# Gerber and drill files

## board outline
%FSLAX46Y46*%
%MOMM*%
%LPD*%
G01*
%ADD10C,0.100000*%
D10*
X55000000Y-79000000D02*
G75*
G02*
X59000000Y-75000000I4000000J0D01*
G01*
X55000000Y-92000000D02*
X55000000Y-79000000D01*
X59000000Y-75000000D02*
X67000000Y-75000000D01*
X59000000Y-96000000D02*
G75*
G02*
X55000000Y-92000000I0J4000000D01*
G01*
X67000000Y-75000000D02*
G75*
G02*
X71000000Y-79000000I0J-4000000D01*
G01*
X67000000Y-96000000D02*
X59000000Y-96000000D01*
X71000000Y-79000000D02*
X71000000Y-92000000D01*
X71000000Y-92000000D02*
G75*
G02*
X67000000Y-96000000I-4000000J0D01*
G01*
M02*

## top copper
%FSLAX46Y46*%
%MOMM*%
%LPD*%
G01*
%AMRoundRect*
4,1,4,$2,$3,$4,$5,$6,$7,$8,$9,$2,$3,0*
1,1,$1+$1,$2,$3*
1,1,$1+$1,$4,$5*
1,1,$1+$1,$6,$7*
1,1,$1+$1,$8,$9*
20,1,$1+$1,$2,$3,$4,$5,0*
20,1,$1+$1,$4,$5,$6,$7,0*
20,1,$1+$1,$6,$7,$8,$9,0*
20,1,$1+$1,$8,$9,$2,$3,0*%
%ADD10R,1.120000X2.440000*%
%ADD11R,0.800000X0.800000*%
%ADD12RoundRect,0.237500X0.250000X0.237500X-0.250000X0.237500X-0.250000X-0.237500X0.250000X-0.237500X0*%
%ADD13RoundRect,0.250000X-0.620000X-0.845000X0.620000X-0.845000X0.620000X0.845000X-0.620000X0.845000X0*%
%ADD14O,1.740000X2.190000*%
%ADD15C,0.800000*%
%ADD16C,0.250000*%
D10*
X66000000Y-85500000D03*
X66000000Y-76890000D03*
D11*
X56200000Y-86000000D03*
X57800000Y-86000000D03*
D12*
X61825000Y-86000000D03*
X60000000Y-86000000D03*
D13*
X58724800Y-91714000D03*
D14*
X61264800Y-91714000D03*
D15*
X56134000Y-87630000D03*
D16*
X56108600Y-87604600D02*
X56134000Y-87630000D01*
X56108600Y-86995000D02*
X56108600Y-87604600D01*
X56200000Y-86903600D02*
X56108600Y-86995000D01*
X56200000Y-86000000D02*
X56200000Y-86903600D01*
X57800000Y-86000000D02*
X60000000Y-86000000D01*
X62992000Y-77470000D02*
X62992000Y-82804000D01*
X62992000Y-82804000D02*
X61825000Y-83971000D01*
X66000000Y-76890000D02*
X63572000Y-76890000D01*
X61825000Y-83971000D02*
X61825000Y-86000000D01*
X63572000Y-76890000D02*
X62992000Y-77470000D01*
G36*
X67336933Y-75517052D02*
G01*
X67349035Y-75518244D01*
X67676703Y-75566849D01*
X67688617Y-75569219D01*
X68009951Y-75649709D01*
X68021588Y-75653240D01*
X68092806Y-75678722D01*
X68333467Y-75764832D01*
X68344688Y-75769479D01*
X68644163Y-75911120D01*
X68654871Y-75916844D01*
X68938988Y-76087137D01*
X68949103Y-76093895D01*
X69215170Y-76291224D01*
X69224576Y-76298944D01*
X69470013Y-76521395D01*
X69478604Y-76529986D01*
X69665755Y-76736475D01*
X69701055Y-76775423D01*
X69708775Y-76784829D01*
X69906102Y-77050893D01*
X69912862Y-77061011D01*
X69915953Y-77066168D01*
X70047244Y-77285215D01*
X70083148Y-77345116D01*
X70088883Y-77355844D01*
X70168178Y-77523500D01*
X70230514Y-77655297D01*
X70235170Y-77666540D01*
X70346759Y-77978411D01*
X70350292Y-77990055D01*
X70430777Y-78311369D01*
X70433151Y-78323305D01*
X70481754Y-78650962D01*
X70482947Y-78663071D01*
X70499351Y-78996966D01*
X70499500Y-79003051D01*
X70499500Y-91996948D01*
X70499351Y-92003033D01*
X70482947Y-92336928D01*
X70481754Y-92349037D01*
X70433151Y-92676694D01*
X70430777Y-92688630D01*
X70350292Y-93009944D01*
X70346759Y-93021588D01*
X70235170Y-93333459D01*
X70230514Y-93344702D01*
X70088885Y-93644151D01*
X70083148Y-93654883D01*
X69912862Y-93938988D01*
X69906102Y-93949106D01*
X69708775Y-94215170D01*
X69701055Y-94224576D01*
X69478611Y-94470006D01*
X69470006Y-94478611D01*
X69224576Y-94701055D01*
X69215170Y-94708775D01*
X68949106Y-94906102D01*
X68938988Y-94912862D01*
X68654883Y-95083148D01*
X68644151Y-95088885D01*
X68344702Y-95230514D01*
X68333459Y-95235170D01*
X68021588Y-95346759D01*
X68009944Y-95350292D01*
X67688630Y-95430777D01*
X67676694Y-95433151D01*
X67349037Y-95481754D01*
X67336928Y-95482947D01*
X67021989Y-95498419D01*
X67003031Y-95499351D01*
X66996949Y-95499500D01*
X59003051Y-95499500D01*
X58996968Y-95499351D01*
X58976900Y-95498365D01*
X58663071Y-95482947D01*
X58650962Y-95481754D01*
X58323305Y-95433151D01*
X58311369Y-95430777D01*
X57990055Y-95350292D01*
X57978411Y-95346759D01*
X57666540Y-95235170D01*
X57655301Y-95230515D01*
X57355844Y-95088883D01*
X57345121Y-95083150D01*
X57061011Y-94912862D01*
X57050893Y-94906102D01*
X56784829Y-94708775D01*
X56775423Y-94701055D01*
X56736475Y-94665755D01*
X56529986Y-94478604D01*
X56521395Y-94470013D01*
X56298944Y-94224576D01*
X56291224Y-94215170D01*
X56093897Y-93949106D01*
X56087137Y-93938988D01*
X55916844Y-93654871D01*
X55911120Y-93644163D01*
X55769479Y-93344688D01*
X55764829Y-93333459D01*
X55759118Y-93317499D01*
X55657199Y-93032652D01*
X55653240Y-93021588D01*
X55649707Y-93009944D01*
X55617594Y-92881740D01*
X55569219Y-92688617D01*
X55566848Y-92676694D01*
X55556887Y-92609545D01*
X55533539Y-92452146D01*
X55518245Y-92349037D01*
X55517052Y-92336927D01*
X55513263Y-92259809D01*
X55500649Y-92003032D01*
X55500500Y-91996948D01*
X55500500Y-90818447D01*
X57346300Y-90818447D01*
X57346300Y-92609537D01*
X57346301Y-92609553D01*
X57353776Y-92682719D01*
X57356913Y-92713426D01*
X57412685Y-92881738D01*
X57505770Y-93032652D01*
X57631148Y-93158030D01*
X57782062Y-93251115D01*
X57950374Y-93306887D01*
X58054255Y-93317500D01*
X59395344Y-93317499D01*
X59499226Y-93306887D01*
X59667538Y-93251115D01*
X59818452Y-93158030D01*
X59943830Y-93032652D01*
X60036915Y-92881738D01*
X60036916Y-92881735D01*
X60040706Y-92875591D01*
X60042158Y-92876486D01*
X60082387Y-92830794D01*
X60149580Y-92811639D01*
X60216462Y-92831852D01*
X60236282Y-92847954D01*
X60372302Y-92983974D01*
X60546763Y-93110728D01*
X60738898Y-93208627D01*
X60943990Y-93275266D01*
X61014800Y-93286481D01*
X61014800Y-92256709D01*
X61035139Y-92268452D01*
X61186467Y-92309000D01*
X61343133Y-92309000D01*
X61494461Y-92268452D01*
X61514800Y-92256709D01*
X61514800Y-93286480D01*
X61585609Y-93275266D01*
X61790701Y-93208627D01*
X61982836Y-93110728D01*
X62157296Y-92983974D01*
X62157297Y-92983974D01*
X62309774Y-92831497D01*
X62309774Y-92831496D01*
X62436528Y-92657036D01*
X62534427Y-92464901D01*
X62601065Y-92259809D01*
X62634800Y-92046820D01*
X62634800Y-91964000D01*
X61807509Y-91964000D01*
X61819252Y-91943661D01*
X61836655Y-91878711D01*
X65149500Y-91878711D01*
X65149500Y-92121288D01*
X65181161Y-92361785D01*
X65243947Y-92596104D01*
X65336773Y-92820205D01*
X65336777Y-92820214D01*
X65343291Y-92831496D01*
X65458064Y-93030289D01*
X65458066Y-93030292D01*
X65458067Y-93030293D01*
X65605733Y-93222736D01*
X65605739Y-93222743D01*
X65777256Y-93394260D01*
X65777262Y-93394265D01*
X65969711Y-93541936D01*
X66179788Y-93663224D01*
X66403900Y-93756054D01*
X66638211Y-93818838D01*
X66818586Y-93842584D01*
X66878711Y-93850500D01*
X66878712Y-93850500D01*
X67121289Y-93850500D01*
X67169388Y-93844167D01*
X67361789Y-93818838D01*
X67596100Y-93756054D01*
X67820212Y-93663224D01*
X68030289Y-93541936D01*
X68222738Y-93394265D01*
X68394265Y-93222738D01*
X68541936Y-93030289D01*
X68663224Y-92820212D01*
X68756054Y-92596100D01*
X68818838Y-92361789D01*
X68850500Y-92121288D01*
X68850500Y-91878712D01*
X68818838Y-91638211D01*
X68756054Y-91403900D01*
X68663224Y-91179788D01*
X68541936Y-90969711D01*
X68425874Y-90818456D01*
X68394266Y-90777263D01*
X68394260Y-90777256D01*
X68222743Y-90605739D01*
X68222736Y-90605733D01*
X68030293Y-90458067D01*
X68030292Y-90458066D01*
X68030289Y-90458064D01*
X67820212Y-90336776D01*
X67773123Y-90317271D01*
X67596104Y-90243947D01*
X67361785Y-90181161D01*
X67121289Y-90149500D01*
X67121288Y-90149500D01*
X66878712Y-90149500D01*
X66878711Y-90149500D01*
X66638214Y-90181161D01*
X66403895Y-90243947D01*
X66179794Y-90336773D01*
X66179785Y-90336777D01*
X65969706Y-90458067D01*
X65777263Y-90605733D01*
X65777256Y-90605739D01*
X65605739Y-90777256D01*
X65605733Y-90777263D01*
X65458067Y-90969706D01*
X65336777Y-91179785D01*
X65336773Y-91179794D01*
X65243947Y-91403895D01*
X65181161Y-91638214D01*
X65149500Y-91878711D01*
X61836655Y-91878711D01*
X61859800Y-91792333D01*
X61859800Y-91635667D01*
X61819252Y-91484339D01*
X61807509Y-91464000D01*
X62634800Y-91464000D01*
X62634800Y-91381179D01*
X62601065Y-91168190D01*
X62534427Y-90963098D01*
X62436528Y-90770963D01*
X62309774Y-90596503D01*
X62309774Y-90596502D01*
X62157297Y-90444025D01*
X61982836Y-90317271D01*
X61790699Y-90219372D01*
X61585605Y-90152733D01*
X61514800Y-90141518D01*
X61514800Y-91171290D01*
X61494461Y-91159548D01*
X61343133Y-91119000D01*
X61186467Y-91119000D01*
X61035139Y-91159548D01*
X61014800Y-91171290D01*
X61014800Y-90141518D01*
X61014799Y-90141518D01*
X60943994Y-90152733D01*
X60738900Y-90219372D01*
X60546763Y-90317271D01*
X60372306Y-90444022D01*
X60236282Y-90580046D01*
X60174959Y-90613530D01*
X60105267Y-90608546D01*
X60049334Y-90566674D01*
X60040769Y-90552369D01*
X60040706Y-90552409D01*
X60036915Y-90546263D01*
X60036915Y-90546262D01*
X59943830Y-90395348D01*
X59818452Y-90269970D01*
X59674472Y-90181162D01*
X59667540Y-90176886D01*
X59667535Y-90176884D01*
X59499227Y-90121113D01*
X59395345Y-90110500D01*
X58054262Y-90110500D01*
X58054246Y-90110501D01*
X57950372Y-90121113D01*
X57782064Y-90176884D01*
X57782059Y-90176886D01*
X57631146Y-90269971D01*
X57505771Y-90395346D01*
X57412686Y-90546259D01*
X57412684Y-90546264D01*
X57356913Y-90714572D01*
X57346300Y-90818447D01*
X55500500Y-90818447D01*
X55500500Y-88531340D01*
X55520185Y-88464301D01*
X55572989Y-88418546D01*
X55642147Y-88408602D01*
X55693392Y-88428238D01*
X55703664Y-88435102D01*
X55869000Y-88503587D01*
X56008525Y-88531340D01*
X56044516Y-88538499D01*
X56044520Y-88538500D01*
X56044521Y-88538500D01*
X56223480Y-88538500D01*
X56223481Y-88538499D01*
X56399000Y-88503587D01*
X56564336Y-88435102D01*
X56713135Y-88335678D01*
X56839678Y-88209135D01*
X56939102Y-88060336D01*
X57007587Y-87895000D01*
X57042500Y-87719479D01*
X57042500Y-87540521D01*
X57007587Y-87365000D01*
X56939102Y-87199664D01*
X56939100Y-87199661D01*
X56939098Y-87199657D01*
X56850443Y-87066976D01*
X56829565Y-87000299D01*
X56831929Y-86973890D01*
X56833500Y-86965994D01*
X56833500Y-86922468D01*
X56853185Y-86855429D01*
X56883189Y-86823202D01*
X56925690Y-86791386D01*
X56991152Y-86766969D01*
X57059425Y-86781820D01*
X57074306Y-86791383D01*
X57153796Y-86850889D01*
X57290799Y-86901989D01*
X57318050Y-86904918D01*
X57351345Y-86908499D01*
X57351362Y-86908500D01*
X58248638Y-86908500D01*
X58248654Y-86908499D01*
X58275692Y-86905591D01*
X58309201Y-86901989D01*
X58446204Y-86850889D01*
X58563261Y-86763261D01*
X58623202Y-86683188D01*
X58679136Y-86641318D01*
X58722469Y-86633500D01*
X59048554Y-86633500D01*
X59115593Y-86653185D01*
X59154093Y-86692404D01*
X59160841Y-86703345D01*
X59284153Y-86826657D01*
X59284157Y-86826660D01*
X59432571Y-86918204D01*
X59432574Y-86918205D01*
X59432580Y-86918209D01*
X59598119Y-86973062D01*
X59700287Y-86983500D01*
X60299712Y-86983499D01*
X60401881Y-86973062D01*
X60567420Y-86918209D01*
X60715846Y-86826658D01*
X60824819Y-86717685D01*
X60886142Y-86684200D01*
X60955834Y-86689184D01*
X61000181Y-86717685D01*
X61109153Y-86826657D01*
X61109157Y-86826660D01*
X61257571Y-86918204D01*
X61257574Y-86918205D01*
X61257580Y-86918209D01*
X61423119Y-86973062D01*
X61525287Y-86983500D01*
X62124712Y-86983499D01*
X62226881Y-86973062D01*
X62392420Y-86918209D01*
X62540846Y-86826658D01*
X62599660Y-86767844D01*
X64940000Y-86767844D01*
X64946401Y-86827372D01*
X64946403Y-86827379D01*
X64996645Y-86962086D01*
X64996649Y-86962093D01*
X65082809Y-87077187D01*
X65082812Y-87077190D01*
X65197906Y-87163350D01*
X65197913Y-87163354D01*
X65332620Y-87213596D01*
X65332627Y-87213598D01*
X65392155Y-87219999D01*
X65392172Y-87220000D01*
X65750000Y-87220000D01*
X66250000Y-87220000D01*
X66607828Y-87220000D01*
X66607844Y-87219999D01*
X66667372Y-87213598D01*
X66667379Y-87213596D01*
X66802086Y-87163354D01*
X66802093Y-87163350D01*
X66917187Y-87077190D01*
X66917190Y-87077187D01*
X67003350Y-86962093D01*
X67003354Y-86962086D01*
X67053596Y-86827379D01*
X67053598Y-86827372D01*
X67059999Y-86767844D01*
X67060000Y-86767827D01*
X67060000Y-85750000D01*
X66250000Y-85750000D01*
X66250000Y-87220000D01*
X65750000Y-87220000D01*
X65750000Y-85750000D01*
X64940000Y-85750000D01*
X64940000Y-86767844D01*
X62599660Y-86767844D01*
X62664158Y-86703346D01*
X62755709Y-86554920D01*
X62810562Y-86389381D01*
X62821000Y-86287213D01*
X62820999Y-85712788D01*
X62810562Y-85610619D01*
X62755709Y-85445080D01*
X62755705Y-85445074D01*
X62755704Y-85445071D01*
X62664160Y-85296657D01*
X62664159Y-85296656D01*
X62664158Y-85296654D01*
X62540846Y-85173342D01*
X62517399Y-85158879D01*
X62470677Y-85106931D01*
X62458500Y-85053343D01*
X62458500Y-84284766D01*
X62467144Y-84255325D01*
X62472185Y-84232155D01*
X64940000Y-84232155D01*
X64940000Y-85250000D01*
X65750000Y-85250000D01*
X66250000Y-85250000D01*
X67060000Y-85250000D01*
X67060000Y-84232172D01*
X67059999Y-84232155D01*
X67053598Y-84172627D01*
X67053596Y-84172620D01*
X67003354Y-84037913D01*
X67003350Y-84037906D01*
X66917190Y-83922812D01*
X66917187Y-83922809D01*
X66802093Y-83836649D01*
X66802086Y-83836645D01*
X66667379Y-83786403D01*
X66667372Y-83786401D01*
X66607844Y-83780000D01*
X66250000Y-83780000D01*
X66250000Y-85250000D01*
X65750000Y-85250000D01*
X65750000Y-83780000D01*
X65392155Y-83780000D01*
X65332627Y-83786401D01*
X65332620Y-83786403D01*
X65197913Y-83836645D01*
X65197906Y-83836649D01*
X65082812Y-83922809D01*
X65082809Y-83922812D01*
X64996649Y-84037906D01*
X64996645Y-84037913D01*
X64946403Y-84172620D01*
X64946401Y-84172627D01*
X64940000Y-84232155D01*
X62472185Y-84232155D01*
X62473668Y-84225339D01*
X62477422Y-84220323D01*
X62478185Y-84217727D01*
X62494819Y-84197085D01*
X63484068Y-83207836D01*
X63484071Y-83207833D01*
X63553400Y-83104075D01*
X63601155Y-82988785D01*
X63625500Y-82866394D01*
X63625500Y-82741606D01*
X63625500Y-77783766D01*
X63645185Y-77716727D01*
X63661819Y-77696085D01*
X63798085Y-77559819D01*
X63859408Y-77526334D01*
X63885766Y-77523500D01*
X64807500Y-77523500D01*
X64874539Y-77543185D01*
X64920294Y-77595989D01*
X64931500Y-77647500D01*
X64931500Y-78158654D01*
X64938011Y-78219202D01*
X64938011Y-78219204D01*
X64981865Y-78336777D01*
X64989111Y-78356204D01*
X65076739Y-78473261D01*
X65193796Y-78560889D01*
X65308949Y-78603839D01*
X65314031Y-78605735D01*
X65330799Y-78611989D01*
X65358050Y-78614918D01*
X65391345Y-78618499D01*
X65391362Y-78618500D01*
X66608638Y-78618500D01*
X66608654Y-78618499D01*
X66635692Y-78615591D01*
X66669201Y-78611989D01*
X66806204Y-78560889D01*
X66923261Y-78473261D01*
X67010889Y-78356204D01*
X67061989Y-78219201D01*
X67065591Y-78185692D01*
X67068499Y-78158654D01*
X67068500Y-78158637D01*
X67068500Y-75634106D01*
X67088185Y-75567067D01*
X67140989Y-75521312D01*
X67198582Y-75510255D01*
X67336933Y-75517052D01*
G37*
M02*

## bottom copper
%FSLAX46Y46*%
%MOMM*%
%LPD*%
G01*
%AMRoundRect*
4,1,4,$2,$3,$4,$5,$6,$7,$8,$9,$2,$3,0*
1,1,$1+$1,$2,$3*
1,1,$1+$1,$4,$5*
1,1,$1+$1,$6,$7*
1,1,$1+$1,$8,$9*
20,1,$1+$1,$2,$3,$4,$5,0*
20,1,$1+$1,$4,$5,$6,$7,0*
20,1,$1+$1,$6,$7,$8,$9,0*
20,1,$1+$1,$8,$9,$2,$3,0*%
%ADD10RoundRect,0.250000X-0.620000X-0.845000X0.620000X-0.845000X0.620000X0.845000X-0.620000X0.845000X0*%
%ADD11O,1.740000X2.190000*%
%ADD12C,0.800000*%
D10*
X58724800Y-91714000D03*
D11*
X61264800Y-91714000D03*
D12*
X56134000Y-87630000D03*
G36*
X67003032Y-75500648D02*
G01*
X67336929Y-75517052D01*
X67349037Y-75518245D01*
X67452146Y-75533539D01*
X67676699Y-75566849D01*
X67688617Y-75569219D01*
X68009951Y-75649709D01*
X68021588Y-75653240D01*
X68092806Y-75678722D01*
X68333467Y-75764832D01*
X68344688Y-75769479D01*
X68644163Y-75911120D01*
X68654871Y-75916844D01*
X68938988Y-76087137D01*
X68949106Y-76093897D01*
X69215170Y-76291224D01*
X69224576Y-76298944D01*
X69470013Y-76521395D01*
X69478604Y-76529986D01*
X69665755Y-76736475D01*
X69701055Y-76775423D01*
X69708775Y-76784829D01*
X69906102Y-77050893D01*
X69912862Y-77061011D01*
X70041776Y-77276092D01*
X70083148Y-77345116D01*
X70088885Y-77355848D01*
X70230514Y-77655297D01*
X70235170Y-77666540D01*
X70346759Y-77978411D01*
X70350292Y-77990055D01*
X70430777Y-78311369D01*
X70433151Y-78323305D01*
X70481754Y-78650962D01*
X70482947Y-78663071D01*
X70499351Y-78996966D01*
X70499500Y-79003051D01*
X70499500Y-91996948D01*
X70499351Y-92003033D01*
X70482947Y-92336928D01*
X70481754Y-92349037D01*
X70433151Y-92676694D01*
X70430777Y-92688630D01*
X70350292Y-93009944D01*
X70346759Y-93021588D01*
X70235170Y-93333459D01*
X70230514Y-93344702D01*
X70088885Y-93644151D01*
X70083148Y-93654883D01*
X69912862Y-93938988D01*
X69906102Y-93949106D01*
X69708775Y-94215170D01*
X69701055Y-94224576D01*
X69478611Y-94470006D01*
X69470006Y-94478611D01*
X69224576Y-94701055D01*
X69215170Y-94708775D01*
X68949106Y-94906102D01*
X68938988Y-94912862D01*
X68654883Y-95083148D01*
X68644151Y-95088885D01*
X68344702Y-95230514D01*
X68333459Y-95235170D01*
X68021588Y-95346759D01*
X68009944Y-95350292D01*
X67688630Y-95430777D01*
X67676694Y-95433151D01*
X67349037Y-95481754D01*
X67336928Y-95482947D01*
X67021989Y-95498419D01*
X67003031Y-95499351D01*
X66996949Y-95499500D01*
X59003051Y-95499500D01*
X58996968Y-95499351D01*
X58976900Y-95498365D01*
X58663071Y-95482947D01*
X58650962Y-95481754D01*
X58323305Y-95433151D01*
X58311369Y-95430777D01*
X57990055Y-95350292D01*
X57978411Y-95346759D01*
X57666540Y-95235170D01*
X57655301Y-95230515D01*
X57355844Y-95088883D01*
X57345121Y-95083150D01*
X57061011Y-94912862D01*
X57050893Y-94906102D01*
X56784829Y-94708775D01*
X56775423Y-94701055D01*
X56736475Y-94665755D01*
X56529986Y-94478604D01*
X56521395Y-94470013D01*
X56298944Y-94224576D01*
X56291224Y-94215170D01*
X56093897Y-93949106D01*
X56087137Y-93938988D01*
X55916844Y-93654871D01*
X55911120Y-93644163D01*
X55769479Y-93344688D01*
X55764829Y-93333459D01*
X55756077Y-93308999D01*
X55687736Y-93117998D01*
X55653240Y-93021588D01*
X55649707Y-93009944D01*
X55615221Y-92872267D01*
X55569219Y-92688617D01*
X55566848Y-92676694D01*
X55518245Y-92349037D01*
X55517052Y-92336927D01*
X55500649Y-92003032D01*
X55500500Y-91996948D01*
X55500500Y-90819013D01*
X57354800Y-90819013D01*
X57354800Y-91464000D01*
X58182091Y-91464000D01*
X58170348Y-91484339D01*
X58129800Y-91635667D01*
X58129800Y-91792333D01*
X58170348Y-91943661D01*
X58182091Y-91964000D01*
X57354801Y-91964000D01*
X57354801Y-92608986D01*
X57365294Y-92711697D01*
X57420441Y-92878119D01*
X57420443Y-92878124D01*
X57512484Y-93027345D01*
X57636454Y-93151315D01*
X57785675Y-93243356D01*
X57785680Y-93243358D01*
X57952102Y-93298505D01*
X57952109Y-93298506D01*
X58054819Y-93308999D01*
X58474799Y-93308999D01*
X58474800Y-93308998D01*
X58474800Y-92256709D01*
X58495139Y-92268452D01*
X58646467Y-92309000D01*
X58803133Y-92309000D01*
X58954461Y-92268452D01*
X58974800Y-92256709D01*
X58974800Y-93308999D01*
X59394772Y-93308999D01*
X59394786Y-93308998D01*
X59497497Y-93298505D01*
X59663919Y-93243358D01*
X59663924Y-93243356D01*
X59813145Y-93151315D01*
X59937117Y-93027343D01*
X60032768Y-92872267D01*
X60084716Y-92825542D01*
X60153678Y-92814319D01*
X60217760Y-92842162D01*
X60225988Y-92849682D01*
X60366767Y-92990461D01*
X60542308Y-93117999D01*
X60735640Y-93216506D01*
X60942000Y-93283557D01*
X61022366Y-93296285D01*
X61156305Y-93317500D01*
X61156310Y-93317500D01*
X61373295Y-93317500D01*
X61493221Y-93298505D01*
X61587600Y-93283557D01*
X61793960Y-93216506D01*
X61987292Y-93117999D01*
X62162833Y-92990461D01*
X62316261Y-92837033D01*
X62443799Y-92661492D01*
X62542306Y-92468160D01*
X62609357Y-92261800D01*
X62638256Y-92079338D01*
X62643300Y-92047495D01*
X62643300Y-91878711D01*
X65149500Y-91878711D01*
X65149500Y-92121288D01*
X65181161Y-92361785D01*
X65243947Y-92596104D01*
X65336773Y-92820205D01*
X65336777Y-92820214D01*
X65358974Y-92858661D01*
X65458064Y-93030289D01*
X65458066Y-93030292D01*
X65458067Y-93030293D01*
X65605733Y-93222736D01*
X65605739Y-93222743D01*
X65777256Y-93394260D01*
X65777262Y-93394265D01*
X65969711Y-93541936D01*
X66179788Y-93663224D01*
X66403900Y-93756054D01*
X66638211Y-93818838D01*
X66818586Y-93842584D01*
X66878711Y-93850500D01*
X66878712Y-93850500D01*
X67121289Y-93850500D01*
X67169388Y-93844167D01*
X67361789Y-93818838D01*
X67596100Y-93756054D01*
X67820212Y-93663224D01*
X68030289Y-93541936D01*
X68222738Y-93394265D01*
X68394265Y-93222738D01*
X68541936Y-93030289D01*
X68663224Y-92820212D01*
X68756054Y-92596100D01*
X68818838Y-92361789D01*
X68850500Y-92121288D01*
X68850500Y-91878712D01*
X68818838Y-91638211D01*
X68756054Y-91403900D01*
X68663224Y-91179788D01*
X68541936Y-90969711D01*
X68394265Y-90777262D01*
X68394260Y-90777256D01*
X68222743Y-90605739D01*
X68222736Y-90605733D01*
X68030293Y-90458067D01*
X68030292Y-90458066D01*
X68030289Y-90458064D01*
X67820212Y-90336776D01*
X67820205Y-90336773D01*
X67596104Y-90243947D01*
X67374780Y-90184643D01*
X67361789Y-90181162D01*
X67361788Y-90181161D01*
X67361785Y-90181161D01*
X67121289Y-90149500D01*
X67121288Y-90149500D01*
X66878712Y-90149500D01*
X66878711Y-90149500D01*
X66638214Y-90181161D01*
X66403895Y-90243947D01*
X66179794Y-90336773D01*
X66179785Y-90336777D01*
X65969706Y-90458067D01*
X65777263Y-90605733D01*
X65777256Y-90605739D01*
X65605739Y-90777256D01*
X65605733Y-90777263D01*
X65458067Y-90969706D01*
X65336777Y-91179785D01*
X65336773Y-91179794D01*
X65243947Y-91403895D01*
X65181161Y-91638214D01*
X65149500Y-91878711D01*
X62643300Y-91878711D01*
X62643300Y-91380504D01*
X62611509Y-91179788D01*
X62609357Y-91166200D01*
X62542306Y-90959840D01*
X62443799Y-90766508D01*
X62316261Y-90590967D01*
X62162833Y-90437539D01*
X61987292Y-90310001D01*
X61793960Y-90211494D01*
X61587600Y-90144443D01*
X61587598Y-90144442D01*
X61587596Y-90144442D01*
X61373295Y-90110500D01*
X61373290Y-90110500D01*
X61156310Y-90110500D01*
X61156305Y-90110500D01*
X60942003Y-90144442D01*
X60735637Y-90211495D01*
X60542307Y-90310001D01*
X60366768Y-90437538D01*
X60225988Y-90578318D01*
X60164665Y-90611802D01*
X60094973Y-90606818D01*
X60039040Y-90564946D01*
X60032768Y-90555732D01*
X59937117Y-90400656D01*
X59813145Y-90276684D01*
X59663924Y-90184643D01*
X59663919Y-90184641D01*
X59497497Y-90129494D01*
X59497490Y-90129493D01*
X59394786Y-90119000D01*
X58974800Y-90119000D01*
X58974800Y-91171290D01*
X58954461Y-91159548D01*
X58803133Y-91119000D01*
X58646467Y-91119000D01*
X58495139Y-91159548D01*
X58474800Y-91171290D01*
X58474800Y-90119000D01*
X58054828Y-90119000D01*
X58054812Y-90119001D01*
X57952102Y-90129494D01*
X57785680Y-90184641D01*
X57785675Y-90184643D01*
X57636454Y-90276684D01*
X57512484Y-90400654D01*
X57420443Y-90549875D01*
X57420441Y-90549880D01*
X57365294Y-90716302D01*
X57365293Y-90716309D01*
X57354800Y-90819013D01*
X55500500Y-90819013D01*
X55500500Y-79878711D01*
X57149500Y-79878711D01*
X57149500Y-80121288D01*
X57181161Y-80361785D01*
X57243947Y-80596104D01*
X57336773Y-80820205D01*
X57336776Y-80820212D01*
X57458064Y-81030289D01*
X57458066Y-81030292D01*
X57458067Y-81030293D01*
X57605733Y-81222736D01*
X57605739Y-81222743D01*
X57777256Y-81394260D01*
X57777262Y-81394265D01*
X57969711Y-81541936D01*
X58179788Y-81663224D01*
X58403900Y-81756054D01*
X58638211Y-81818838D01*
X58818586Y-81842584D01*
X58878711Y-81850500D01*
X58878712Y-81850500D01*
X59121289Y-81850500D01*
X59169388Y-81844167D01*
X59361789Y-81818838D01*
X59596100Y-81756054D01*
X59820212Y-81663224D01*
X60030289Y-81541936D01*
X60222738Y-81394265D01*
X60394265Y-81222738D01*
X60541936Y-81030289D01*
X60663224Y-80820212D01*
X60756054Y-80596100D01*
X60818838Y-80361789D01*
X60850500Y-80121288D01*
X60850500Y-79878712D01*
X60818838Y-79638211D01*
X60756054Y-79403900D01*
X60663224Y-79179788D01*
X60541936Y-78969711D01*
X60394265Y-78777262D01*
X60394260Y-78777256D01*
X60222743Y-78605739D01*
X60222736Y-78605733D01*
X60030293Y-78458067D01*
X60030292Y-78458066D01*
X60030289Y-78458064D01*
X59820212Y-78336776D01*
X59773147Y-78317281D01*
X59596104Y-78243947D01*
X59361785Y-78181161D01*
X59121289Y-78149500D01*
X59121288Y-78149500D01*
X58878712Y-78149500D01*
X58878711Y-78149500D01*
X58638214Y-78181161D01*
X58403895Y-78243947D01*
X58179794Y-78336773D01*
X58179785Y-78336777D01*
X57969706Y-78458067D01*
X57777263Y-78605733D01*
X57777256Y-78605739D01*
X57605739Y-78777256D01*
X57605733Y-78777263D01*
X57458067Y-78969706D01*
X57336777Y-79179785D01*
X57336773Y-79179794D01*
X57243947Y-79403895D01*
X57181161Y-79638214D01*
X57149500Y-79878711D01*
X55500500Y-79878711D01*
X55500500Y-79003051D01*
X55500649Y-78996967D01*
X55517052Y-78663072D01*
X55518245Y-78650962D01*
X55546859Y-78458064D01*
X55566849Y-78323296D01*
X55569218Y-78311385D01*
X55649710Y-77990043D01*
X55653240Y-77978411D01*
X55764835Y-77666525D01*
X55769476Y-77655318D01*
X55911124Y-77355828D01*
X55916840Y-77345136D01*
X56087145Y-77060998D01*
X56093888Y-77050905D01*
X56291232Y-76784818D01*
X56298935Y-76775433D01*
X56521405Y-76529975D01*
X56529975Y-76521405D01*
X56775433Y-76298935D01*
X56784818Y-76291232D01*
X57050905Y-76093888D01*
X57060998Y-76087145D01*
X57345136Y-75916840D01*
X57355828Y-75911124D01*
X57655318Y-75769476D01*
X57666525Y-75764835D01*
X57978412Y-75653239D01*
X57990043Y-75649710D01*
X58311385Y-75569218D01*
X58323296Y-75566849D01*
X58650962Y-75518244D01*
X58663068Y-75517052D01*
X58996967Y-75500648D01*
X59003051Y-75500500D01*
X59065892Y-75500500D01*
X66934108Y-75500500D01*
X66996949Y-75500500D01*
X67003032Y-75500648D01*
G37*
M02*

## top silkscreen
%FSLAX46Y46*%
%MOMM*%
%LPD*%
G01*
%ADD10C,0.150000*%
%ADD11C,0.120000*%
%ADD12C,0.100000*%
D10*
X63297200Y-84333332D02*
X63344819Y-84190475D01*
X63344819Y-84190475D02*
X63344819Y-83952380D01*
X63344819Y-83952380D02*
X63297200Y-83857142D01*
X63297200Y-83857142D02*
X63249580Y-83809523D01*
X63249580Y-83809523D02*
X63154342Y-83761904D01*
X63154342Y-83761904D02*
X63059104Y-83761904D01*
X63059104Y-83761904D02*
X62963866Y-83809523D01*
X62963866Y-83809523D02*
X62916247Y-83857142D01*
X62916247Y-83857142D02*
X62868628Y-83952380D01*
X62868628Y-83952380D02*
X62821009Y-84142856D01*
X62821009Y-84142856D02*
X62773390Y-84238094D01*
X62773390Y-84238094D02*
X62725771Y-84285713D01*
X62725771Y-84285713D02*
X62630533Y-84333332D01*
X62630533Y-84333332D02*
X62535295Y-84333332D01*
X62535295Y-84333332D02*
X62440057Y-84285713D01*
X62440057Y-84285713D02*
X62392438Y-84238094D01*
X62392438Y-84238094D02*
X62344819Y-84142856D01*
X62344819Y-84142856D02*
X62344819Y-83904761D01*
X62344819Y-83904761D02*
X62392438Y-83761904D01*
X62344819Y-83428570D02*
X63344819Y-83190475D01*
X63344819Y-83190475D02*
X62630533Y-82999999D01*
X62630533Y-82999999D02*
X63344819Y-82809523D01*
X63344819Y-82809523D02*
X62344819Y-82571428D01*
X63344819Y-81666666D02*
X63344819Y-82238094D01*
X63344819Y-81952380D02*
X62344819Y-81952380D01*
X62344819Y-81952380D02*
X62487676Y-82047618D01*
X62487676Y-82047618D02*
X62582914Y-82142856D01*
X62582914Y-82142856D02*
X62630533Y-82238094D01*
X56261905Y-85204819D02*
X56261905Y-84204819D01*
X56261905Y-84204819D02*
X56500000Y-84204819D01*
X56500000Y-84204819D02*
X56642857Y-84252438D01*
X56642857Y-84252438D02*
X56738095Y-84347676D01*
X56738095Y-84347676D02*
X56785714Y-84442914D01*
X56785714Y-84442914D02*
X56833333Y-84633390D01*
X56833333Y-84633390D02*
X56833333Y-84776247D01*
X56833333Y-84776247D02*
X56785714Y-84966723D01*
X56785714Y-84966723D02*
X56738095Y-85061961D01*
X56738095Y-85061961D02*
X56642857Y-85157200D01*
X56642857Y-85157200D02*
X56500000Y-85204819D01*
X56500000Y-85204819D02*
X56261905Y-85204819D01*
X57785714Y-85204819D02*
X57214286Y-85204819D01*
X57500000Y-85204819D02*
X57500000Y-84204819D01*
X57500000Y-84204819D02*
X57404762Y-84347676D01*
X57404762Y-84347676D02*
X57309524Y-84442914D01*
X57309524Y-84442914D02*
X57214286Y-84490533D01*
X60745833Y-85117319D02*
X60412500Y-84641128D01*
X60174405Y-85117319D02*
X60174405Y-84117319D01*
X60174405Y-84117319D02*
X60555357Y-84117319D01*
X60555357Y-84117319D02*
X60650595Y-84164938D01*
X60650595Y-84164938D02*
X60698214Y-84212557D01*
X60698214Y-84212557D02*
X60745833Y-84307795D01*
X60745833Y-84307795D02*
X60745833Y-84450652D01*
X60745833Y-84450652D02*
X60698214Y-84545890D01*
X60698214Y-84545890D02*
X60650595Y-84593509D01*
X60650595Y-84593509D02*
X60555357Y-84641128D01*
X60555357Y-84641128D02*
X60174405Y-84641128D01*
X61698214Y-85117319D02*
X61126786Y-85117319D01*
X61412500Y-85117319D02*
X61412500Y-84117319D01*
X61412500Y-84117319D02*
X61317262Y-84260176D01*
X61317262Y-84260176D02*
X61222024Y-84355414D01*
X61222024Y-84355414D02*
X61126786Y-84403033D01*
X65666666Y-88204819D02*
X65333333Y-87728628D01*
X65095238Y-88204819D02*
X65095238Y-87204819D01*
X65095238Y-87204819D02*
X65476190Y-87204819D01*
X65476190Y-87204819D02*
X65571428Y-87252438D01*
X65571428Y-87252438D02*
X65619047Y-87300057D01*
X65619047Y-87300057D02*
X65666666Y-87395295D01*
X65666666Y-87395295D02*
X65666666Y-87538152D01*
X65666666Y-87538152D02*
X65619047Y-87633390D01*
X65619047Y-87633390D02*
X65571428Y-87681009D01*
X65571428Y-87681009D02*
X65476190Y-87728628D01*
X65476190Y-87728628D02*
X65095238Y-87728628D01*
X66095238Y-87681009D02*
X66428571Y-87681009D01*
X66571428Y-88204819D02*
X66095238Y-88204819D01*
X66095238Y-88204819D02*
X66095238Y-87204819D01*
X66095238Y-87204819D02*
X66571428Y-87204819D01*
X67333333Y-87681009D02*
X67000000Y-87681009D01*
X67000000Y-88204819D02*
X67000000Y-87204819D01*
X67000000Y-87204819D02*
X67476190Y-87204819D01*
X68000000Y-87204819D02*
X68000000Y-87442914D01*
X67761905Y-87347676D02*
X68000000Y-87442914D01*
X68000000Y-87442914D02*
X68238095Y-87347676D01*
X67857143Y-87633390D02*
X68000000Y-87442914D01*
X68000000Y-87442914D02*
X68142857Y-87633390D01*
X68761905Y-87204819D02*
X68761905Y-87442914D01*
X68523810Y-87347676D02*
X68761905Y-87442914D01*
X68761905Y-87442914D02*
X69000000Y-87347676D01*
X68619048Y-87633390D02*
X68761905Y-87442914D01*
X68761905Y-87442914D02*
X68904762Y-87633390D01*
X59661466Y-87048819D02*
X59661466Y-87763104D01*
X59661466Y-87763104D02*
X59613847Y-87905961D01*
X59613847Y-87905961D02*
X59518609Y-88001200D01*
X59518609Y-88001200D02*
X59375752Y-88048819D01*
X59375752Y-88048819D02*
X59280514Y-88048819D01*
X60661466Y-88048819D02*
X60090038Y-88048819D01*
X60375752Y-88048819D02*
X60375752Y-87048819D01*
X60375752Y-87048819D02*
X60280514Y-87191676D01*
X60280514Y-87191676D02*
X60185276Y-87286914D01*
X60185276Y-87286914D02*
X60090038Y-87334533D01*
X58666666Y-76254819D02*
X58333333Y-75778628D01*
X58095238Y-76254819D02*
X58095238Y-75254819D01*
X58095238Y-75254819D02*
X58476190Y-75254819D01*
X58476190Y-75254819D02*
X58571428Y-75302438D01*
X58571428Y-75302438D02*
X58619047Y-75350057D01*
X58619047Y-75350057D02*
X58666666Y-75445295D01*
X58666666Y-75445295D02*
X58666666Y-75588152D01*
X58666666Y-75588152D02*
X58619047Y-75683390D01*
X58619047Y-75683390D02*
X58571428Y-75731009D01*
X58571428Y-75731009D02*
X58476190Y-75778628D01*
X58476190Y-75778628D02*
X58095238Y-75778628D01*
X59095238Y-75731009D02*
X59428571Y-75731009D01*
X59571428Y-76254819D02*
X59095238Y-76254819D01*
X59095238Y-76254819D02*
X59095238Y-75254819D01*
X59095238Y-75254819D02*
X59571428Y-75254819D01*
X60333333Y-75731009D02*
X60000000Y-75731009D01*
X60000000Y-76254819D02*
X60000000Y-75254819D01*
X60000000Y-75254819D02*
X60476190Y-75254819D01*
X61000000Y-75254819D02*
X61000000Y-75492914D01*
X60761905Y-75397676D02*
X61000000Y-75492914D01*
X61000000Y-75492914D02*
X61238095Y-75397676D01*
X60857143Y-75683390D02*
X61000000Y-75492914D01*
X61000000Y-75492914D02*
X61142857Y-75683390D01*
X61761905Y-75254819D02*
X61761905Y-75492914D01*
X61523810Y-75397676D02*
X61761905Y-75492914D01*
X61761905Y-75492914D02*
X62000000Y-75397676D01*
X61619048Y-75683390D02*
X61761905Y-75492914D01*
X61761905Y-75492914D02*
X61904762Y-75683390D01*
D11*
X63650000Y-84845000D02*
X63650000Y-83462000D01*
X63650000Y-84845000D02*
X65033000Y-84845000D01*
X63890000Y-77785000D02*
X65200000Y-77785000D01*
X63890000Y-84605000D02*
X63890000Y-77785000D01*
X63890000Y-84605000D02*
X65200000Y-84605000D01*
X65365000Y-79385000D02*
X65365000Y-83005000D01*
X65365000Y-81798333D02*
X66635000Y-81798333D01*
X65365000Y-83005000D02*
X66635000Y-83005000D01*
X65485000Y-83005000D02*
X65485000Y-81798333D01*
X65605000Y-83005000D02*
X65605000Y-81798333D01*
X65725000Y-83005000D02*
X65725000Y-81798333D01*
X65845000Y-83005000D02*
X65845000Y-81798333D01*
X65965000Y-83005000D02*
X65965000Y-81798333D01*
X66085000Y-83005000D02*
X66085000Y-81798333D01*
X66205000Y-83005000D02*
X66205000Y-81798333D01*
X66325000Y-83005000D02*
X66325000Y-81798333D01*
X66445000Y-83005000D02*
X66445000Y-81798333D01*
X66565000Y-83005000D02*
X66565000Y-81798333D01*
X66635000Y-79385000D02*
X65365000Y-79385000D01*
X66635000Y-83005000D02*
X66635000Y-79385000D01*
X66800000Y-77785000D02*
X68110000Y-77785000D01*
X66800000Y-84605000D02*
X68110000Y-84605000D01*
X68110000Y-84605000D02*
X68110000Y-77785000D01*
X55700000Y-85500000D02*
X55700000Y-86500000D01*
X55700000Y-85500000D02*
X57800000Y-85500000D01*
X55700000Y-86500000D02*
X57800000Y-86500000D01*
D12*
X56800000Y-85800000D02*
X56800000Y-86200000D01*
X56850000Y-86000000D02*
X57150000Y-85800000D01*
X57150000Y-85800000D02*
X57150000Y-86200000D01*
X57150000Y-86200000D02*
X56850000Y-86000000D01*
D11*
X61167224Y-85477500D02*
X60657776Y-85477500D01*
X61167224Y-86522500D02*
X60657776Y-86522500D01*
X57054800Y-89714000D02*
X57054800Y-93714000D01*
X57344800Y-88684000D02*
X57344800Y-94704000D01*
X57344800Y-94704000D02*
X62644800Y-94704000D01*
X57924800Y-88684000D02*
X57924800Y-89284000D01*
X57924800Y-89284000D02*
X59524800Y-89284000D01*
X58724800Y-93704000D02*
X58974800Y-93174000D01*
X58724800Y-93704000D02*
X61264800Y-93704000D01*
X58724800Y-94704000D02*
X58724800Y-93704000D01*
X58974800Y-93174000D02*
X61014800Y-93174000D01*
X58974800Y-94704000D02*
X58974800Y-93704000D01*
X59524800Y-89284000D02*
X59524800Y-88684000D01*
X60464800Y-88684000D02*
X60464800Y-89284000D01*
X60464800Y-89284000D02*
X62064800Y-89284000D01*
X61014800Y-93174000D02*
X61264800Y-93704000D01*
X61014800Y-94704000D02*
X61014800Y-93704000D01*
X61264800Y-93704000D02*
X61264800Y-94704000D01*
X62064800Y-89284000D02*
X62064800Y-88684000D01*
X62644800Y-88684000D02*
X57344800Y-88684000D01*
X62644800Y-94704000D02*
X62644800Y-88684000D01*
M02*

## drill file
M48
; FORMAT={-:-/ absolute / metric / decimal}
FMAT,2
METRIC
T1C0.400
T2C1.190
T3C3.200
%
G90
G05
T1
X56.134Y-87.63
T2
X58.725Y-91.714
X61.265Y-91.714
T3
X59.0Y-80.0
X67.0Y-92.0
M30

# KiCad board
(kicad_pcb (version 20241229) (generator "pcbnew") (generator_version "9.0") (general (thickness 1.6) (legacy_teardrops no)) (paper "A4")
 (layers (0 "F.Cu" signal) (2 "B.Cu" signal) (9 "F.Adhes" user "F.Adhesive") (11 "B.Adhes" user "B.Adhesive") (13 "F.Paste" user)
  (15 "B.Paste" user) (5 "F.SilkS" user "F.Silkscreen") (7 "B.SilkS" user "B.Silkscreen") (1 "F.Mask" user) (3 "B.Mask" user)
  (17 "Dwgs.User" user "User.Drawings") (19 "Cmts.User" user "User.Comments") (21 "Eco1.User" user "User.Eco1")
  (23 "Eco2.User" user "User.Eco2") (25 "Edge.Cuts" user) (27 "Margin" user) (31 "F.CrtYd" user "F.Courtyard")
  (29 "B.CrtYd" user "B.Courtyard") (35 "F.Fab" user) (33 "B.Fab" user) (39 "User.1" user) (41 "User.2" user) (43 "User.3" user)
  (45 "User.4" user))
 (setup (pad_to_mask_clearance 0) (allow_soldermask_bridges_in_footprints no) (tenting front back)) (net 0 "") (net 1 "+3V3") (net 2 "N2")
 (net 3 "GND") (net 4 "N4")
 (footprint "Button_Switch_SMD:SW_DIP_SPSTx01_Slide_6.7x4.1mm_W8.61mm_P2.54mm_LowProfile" (layer "F.Cu") (at 66 81.195 90)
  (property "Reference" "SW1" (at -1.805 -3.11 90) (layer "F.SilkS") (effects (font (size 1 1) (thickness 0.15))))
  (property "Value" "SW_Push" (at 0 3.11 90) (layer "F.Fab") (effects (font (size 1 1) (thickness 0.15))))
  (fp_line (start -3.65 -2.35) (end -2.267 -2.35) (stroke (width 0.12) (type solid)) (layer "F.SilkS"))
  (fp_line (start -3.65 -2.35) (end -3.65 -0.967) (stroke (width 0.12) (type solid)) (layer "F.SilkS"))
  (fp_line (start 3.41 -2.11) (end 3.41 -0.8) (stroke (width 0.12) (type solid)) (layer "F.SilkS"))
  (fp_line (start -3.41 -2.11) (end 3.41 -2.11) (stroke (width 0.12) (type solid)) (layer "F.SilkS"))
  (fp_line (start -3.41 -2.11) (end -3.41 -0.8) (stroke (width 0.12) (type solid)) (layer "F.SilkS"))
  (fp_line (start 1.81 -0.635) (end -1.81 -0.635) (stroke (width 0.12) (type solid)) (layer "F.SilkS"))
  (fp_line (start -0.603333 -0.635) (end -0.603333 0.635) (stroke (width 0.12) (type solid)) (layer "F.SilkS"))
  (fp_line (start -1.81 -0.635) (end -1.81 0.635) (stroke (width 0.12) (type solid)) (layer "F.SilkS"))
  (fp_line (start -1.81 -0.515) (end -0.603333 -0.515) (stroke (width 0.12) (type solid)) (layer "F.SilkS"))
  (fp_line (start -1.81 -0.395) (end -0.603333 -0.395) (stroke (width 0.12) (type solid)) (layer "F.SilkS"))
  (fp_line (start -1.81 -0.275) (end -0.603333 -0.275) (stroke (width 0.12) (type solid)) (layer "F.SilkS"))
  (fp_line (start -1.81 -0.155) (end -0.603333 -0.155) (stroke (width 0.12) (type solid)) (layer "F.SilkS"))
  (fp_line (start -1.81 -0.035) (end -0.603333 -0.035) (stroke (width 0.12) (type solid)) (layer "F.SilkS"))
  (fp_line (start -1.81 0.085) (end -0.603333 0.085) (stroke (width 0.12) (type solid)) (layer "F.SilkS"))
  (fp_line (start -1.81 0.205) (end -0.603333 0.205) (stroke (width 0.12) (type solid)) (layer "F.SilkS"))
  (fp_line (start -1.81 0.325) (end -0.603333 0.325) (stroke (width 0.12) (type solid)) (layer "F.SilkS"))
  (fp_line (start -1.81 0.445) (end -0.603333 0.445) (stroke (width 0.12) (type solid)) (layer "F.SilkS"))
  (fp_line (start -1.81 0.565) (end -0.603333 0.565) (stroke (width 0.12) (type solid)) (layer "F.SilkS"))
  (fp_line (start 1.81 0.635) (end 1.81 -0.635) (stroke (width 0.12) (type solid)) (layer "F.SilkS"))
  (fp_line (start -1.81 0.635) (end 1.81 0.635) (stroke (width 0.12) (type solid)) (layer "F.SilkS"))
  (fp_line (start 3.41 0.8) (end 3.41 2.11) (stroke (width 0.12) (type solid)) (layer "F.SilkS"))
  (fp_line (start -3.41 0.8) (end -3.41 2.11) (stroke (width 0.12) (type solid)) (layer "F.SilkS"))
  (fp_line (start -3.41 2.11) (end 3.41 2.11) (stroke (width 0.12) (type solid)) (layer "F.SilkS"))
  (pad "1" smd rect (at -4.305 0 90) (size 2.44 1.12) (layers "F.Cu" "F.Mask" "F.Paste") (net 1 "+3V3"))
  (pad "2" smd rect (at 4.305 0 90) (size 2.44 1.12) (layers "F.Cu" "F.Mask" "F.Paste") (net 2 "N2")))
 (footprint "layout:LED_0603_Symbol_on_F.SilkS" (layer "F.Cu") (at 57 86)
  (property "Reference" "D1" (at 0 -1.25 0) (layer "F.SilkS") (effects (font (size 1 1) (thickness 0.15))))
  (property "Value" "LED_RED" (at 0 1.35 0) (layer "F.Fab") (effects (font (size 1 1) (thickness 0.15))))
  (fp_line (start -1.3 -0.5) (end -1.3 0.5) (stroke (width 0.12) (type solid)) (layer "F.SilkS"))
  (fp_line (start -1.3 -0.5) (end 0.8 -0.5) (stroke (width 0.12) (type solid)) (layer "F.SilkS"))
  (fp_line (start -1.3 0.5) (end 0.8 0.5) (stroke (width 0.12) (type solid)) (layer "F.SilkS"))
  (fp_line (start -0.2 -0.2) (end -0.2 0.2) (stroke (width 0.1) (type solid)) (layer "F.SilkS"))
  (fp_line (start -0.15 0) (end 0.15 -0.2) (stroke (width 0.1) (type solid)) (layer "F.SilkS"))
  (fp_line (start 0.15 -0.2) (end 0.15 0.2) (stroke (width 0.1) (type solid)) (layer "F.SilkS"))
  (fp_line (start 0.15 0.2) (end -0.15 0) (stroke (width 0.1) (type solid)) (layer "F.SilkS"))
  (pad "1" smd rect (at -0.8 0 180) (size 0.8 0.8) (layers "F.Cu" "F.Mask" "F.Paste") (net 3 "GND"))
  (pad "2" smd rect (at 0.8 0 180) (size 0.8 0.8) (layers "F.Cu" "F.Mask" "F.Paste") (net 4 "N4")))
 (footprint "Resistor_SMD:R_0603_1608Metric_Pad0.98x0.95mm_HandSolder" (layer "F.Cu") (at 60.9125 86 180)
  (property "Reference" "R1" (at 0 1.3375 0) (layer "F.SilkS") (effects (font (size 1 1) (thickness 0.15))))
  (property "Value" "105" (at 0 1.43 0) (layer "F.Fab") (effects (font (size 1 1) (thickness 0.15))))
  (fp_line (start -0.254724 0.5225) (end 0.254724 0.5225) (stroke (width 0.12) (type solid)) (layer "F.SilkS"))
  (fp_line (start -0.254724 -0.5225) (end 0.254724 -0.5225) (stroke (width 0.12) (type solid)) (layer "F.SilkS"))
  (pad "1" smd roundrect (at -0.9125 0 180) (size 0.975 0.95) (layers "F.Cu" "F.Mask" "F.Paste") (roundrect_rratio 0.25) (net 2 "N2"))
  (pad "2" smd roundrect (at 0.9125 0 180) (size 0.975 0.95) (layers "F.Cu" "F.Mask" "F.Paste") (roundrect_rratio 0.25) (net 4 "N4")))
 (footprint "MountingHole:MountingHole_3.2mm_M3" (layer "F.Cu") (at 67 92 180)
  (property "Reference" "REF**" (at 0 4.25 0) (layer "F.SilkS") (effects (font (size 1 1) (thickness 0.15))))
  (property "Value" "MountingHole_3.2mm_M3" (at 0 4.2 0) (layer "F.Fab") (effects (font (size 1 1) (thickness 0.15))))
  (pad "" np_thru_hole circle (at 0 0 180) (size 3.2 3.2) (drill 3.2) (layers "*.Cu" "*.Mask")))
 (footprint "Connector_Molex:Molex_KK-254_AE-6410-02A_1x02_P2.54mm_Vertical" (layer "F.Cu") (at 58.7248 91.714)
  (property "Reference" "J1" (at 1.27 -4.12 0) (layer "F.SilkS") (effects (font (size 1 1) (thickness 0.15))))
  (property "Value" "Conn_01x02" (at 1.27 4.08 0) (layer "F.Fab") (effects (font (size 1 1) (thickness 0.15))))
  (fp_line (start -1.67 -2) (end -1.67 2) (stroke (width 0.12) (type solid)) (layer "F.SilkS"))
  (fp_line (start -1.38 -3.03) (end -1.38 2.99) (stroke (width 0.12) (type solid)) (layer "F.SilkS"))
  (fp_line (start -1.38 2.99) (end 3.92 2.99) (stroke (width 0.12) (type solid)) (layer "F.SilkS"))
  (fp_line (start -0.8 -3.03) (end -0.8 -2.43) (stroke (width 0.12) (type solid)) (layer "F.SilkS"))
  (fp_line (start -0.8 -2.43) (end 0.8 -2.43) (stroke (width 0.12) (type solid)) (layer "F.SilkS"))
  (fp_line (start 0 1.99) (end 0.25 1.46) (stroke (width 0.12) (type solid)) (layer "F.SilkS"))
  (fp_line (start 0 1.99) (end 2.54 1.99) (stroke (width 0.12) (type solid)) (layer "F.SilkS"))
  (fp_line (start 0 2.99) (end 0 1.99) (stroke (width 0.12) (type solid)) (layer "F.SilkS"))
  (fp_line (start 0.25 1.46) (end 2.29 1.46) (stroke (width 0.12) (type solid)) (layer "F.SilkS"))
  (fp_line (start 0.25 2.99) (end 0.25 1.99) (stroke (width 0.12) (type solid)) (layer "F.SilkS"))
  (fp_line (start 0.8 -2.43) (end 0.8 -3.03) (stroke (width 0.12) (type solid)) (layer "F.SilkS"))
  (fp_line (start 1.74 -3.03) (end 1.74 -2.43) (stroke (width 0.12) (type solid)) (layer "F.SilkS"))
  (fp_line (start 1.74 -2.43) (end 3.34 -2.43) (stroke (width 0.12) (type solid)) (layer "F.SilkS"))
  (fp_line (start 2.29 1.46) (end 2.54 1.99) (stroke (width 0.12) (type solid)) (layer "F.SilkS"))
  (fp_line (start 2.29 2.99) (end 2.29 1.99) (stroke (width 0.12) (type solid)) (layer "F.SilkS"))
  (fp_line (start 2.54 1.99) (end 2.54 2.99) (stroke (width 0.12) (type solid)) (layer "F.SilkS"))
  (fp_line (start 3.34 -2.43) (end 3.34 -3.03) (stroke (width 0.12) (type solid)) (layer "F.SilkS"))
  (fp_line (start 3.92 -3.03) (end -1.38 -3.03) (stroke (width 0.12) (type solid)) (layer "F.SilkS"))
  (fp_line (start 3.92 2.99) (end 3.92 -3.03) (stroke (width 0.12) (type solid)) (layer "F.SilkS"))
  (pad "1" thru_hole roundrect (at 0 0) (size 1.74 2.19) (drill 1.19) (layers "*.Cu" "*.Mask") (remove_unused_layers no)
   (roundrect_rratio 0.143678) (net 3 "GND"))
  (pad "2" thru_hole oval (at 2.54 0) (size 1.74 2.19) (drill 1.19) (layers "*.Cu" "*.Mask") (remove_unused_layers no) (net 1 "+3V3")))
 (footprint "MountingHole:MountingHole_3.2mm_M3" (layer "F.Cu") (at 59 80)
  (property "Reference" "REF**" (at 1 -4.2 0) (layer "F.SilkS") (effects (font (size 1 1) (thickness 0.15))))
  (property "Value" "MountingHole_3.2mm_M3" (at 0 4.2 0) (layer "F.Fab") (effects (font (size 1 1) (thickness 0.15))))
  (pad "" np_thru_hole circle (at 0 0) (size 3.2 3.2) (drill 3.2) (layers "*.Cu" "*.Mask")))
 (gr_arc (start 55 79) (mid 56.171573 76.171573) (end 59 75) (stroke (width 0.1) (type default)) (layer "Edge.Cuts"))
 (gr_line (start 55 92) (end 55 79) (stroke (width 0.1) (type default)) (layer "Edge.Cuts"))
 (gr_line (start 59 75) (end 67 75) (stroke (width 0.1) (type default)) (layer "Edge.Cuts"))
 (gr_arc (start 59 96) (mid 56.171573 94.828427) (end 55 92) (stroke (width 0.1) (type default)) (layer "Edge.Cuts"))
 (gr_arc (start 67 75) (mid 69.828427 76.171573) (end 71 79) (stroke (width 0.1) (type default)) (layer "Edge.Cuts"))
 (gr_line (start 67 96) (end 59 96) (stroke (width 0.1) (type default)) (layer "Edge.Cuts"))
 (gr_line (start 71 79) (end 71 92) (stroke (width 0.1) (type default)) (layer "Edge.Cuts"))
 (gr_arc (start 71 92) (mid 69.828427 94.828427) (end 67 96) (stroke (width 0.1) (type default)) (layer "Edge.Cuts"))
 (segment (start 56.1086 87.6046) (end 56.134 87.63) (width 0.25) (layer "F.Cu") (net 3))
 (segment (start 56.1086 86.995) (end 56.1086 87.6046) (width 0.25) (layer "F.Cu") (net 3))
 (segment (start 56.2 86.9036) (end 56.1086 86.995) (width 0.25) (layer "F.Cu") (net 3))
 (segment (start 56.2 86) (end 56.2 86.9036) (width 0.25) (layer "F.Cu") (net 3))
 (via (at 56.134 87.63) (size 0.8) (drill 0.4) (layers "F.Cu" "B.Cu") (free yes) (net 3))
 (segment (start 57.8 86) (end 60 86) (width 0.25) (layer "F.Cu") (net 4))
 (segment (start 62.992 77.47) (end 62.992 82.804) (width 0.25) (layer "F.Cu") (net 2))
 (segment (start 62.992 82.804) (end 61.825 83.971) (width 0.25) (layer "F.Cu") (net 2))
 (segment (start 66 76.89) (end 63.572 76.89) (width 0.25) (layer "F.Cu") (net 2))
 (segment (start 61.825 83.971) (end 61.825 86) (width 0.25) (layer "F.Cu") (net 2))
 (segment (start 63.572 76.89) (end 62.992 77.47) (width 0.25) (layer "F.Cu") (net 2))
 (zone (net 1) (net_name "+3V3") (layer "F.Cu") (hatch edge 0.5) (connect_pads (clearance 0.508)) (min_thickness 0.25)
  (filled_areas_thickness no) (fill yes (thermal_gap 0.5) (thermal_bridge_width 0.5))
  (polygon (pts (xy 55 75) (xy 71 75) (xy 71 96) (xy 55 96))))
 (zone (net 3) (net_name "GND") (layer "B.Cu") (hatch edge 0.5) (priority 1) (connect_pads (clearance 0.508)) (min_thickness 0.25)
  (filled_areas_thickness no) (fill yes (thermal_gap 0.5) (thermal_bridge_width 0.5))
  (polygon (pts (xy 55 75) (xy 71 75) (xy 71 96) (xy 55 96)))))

